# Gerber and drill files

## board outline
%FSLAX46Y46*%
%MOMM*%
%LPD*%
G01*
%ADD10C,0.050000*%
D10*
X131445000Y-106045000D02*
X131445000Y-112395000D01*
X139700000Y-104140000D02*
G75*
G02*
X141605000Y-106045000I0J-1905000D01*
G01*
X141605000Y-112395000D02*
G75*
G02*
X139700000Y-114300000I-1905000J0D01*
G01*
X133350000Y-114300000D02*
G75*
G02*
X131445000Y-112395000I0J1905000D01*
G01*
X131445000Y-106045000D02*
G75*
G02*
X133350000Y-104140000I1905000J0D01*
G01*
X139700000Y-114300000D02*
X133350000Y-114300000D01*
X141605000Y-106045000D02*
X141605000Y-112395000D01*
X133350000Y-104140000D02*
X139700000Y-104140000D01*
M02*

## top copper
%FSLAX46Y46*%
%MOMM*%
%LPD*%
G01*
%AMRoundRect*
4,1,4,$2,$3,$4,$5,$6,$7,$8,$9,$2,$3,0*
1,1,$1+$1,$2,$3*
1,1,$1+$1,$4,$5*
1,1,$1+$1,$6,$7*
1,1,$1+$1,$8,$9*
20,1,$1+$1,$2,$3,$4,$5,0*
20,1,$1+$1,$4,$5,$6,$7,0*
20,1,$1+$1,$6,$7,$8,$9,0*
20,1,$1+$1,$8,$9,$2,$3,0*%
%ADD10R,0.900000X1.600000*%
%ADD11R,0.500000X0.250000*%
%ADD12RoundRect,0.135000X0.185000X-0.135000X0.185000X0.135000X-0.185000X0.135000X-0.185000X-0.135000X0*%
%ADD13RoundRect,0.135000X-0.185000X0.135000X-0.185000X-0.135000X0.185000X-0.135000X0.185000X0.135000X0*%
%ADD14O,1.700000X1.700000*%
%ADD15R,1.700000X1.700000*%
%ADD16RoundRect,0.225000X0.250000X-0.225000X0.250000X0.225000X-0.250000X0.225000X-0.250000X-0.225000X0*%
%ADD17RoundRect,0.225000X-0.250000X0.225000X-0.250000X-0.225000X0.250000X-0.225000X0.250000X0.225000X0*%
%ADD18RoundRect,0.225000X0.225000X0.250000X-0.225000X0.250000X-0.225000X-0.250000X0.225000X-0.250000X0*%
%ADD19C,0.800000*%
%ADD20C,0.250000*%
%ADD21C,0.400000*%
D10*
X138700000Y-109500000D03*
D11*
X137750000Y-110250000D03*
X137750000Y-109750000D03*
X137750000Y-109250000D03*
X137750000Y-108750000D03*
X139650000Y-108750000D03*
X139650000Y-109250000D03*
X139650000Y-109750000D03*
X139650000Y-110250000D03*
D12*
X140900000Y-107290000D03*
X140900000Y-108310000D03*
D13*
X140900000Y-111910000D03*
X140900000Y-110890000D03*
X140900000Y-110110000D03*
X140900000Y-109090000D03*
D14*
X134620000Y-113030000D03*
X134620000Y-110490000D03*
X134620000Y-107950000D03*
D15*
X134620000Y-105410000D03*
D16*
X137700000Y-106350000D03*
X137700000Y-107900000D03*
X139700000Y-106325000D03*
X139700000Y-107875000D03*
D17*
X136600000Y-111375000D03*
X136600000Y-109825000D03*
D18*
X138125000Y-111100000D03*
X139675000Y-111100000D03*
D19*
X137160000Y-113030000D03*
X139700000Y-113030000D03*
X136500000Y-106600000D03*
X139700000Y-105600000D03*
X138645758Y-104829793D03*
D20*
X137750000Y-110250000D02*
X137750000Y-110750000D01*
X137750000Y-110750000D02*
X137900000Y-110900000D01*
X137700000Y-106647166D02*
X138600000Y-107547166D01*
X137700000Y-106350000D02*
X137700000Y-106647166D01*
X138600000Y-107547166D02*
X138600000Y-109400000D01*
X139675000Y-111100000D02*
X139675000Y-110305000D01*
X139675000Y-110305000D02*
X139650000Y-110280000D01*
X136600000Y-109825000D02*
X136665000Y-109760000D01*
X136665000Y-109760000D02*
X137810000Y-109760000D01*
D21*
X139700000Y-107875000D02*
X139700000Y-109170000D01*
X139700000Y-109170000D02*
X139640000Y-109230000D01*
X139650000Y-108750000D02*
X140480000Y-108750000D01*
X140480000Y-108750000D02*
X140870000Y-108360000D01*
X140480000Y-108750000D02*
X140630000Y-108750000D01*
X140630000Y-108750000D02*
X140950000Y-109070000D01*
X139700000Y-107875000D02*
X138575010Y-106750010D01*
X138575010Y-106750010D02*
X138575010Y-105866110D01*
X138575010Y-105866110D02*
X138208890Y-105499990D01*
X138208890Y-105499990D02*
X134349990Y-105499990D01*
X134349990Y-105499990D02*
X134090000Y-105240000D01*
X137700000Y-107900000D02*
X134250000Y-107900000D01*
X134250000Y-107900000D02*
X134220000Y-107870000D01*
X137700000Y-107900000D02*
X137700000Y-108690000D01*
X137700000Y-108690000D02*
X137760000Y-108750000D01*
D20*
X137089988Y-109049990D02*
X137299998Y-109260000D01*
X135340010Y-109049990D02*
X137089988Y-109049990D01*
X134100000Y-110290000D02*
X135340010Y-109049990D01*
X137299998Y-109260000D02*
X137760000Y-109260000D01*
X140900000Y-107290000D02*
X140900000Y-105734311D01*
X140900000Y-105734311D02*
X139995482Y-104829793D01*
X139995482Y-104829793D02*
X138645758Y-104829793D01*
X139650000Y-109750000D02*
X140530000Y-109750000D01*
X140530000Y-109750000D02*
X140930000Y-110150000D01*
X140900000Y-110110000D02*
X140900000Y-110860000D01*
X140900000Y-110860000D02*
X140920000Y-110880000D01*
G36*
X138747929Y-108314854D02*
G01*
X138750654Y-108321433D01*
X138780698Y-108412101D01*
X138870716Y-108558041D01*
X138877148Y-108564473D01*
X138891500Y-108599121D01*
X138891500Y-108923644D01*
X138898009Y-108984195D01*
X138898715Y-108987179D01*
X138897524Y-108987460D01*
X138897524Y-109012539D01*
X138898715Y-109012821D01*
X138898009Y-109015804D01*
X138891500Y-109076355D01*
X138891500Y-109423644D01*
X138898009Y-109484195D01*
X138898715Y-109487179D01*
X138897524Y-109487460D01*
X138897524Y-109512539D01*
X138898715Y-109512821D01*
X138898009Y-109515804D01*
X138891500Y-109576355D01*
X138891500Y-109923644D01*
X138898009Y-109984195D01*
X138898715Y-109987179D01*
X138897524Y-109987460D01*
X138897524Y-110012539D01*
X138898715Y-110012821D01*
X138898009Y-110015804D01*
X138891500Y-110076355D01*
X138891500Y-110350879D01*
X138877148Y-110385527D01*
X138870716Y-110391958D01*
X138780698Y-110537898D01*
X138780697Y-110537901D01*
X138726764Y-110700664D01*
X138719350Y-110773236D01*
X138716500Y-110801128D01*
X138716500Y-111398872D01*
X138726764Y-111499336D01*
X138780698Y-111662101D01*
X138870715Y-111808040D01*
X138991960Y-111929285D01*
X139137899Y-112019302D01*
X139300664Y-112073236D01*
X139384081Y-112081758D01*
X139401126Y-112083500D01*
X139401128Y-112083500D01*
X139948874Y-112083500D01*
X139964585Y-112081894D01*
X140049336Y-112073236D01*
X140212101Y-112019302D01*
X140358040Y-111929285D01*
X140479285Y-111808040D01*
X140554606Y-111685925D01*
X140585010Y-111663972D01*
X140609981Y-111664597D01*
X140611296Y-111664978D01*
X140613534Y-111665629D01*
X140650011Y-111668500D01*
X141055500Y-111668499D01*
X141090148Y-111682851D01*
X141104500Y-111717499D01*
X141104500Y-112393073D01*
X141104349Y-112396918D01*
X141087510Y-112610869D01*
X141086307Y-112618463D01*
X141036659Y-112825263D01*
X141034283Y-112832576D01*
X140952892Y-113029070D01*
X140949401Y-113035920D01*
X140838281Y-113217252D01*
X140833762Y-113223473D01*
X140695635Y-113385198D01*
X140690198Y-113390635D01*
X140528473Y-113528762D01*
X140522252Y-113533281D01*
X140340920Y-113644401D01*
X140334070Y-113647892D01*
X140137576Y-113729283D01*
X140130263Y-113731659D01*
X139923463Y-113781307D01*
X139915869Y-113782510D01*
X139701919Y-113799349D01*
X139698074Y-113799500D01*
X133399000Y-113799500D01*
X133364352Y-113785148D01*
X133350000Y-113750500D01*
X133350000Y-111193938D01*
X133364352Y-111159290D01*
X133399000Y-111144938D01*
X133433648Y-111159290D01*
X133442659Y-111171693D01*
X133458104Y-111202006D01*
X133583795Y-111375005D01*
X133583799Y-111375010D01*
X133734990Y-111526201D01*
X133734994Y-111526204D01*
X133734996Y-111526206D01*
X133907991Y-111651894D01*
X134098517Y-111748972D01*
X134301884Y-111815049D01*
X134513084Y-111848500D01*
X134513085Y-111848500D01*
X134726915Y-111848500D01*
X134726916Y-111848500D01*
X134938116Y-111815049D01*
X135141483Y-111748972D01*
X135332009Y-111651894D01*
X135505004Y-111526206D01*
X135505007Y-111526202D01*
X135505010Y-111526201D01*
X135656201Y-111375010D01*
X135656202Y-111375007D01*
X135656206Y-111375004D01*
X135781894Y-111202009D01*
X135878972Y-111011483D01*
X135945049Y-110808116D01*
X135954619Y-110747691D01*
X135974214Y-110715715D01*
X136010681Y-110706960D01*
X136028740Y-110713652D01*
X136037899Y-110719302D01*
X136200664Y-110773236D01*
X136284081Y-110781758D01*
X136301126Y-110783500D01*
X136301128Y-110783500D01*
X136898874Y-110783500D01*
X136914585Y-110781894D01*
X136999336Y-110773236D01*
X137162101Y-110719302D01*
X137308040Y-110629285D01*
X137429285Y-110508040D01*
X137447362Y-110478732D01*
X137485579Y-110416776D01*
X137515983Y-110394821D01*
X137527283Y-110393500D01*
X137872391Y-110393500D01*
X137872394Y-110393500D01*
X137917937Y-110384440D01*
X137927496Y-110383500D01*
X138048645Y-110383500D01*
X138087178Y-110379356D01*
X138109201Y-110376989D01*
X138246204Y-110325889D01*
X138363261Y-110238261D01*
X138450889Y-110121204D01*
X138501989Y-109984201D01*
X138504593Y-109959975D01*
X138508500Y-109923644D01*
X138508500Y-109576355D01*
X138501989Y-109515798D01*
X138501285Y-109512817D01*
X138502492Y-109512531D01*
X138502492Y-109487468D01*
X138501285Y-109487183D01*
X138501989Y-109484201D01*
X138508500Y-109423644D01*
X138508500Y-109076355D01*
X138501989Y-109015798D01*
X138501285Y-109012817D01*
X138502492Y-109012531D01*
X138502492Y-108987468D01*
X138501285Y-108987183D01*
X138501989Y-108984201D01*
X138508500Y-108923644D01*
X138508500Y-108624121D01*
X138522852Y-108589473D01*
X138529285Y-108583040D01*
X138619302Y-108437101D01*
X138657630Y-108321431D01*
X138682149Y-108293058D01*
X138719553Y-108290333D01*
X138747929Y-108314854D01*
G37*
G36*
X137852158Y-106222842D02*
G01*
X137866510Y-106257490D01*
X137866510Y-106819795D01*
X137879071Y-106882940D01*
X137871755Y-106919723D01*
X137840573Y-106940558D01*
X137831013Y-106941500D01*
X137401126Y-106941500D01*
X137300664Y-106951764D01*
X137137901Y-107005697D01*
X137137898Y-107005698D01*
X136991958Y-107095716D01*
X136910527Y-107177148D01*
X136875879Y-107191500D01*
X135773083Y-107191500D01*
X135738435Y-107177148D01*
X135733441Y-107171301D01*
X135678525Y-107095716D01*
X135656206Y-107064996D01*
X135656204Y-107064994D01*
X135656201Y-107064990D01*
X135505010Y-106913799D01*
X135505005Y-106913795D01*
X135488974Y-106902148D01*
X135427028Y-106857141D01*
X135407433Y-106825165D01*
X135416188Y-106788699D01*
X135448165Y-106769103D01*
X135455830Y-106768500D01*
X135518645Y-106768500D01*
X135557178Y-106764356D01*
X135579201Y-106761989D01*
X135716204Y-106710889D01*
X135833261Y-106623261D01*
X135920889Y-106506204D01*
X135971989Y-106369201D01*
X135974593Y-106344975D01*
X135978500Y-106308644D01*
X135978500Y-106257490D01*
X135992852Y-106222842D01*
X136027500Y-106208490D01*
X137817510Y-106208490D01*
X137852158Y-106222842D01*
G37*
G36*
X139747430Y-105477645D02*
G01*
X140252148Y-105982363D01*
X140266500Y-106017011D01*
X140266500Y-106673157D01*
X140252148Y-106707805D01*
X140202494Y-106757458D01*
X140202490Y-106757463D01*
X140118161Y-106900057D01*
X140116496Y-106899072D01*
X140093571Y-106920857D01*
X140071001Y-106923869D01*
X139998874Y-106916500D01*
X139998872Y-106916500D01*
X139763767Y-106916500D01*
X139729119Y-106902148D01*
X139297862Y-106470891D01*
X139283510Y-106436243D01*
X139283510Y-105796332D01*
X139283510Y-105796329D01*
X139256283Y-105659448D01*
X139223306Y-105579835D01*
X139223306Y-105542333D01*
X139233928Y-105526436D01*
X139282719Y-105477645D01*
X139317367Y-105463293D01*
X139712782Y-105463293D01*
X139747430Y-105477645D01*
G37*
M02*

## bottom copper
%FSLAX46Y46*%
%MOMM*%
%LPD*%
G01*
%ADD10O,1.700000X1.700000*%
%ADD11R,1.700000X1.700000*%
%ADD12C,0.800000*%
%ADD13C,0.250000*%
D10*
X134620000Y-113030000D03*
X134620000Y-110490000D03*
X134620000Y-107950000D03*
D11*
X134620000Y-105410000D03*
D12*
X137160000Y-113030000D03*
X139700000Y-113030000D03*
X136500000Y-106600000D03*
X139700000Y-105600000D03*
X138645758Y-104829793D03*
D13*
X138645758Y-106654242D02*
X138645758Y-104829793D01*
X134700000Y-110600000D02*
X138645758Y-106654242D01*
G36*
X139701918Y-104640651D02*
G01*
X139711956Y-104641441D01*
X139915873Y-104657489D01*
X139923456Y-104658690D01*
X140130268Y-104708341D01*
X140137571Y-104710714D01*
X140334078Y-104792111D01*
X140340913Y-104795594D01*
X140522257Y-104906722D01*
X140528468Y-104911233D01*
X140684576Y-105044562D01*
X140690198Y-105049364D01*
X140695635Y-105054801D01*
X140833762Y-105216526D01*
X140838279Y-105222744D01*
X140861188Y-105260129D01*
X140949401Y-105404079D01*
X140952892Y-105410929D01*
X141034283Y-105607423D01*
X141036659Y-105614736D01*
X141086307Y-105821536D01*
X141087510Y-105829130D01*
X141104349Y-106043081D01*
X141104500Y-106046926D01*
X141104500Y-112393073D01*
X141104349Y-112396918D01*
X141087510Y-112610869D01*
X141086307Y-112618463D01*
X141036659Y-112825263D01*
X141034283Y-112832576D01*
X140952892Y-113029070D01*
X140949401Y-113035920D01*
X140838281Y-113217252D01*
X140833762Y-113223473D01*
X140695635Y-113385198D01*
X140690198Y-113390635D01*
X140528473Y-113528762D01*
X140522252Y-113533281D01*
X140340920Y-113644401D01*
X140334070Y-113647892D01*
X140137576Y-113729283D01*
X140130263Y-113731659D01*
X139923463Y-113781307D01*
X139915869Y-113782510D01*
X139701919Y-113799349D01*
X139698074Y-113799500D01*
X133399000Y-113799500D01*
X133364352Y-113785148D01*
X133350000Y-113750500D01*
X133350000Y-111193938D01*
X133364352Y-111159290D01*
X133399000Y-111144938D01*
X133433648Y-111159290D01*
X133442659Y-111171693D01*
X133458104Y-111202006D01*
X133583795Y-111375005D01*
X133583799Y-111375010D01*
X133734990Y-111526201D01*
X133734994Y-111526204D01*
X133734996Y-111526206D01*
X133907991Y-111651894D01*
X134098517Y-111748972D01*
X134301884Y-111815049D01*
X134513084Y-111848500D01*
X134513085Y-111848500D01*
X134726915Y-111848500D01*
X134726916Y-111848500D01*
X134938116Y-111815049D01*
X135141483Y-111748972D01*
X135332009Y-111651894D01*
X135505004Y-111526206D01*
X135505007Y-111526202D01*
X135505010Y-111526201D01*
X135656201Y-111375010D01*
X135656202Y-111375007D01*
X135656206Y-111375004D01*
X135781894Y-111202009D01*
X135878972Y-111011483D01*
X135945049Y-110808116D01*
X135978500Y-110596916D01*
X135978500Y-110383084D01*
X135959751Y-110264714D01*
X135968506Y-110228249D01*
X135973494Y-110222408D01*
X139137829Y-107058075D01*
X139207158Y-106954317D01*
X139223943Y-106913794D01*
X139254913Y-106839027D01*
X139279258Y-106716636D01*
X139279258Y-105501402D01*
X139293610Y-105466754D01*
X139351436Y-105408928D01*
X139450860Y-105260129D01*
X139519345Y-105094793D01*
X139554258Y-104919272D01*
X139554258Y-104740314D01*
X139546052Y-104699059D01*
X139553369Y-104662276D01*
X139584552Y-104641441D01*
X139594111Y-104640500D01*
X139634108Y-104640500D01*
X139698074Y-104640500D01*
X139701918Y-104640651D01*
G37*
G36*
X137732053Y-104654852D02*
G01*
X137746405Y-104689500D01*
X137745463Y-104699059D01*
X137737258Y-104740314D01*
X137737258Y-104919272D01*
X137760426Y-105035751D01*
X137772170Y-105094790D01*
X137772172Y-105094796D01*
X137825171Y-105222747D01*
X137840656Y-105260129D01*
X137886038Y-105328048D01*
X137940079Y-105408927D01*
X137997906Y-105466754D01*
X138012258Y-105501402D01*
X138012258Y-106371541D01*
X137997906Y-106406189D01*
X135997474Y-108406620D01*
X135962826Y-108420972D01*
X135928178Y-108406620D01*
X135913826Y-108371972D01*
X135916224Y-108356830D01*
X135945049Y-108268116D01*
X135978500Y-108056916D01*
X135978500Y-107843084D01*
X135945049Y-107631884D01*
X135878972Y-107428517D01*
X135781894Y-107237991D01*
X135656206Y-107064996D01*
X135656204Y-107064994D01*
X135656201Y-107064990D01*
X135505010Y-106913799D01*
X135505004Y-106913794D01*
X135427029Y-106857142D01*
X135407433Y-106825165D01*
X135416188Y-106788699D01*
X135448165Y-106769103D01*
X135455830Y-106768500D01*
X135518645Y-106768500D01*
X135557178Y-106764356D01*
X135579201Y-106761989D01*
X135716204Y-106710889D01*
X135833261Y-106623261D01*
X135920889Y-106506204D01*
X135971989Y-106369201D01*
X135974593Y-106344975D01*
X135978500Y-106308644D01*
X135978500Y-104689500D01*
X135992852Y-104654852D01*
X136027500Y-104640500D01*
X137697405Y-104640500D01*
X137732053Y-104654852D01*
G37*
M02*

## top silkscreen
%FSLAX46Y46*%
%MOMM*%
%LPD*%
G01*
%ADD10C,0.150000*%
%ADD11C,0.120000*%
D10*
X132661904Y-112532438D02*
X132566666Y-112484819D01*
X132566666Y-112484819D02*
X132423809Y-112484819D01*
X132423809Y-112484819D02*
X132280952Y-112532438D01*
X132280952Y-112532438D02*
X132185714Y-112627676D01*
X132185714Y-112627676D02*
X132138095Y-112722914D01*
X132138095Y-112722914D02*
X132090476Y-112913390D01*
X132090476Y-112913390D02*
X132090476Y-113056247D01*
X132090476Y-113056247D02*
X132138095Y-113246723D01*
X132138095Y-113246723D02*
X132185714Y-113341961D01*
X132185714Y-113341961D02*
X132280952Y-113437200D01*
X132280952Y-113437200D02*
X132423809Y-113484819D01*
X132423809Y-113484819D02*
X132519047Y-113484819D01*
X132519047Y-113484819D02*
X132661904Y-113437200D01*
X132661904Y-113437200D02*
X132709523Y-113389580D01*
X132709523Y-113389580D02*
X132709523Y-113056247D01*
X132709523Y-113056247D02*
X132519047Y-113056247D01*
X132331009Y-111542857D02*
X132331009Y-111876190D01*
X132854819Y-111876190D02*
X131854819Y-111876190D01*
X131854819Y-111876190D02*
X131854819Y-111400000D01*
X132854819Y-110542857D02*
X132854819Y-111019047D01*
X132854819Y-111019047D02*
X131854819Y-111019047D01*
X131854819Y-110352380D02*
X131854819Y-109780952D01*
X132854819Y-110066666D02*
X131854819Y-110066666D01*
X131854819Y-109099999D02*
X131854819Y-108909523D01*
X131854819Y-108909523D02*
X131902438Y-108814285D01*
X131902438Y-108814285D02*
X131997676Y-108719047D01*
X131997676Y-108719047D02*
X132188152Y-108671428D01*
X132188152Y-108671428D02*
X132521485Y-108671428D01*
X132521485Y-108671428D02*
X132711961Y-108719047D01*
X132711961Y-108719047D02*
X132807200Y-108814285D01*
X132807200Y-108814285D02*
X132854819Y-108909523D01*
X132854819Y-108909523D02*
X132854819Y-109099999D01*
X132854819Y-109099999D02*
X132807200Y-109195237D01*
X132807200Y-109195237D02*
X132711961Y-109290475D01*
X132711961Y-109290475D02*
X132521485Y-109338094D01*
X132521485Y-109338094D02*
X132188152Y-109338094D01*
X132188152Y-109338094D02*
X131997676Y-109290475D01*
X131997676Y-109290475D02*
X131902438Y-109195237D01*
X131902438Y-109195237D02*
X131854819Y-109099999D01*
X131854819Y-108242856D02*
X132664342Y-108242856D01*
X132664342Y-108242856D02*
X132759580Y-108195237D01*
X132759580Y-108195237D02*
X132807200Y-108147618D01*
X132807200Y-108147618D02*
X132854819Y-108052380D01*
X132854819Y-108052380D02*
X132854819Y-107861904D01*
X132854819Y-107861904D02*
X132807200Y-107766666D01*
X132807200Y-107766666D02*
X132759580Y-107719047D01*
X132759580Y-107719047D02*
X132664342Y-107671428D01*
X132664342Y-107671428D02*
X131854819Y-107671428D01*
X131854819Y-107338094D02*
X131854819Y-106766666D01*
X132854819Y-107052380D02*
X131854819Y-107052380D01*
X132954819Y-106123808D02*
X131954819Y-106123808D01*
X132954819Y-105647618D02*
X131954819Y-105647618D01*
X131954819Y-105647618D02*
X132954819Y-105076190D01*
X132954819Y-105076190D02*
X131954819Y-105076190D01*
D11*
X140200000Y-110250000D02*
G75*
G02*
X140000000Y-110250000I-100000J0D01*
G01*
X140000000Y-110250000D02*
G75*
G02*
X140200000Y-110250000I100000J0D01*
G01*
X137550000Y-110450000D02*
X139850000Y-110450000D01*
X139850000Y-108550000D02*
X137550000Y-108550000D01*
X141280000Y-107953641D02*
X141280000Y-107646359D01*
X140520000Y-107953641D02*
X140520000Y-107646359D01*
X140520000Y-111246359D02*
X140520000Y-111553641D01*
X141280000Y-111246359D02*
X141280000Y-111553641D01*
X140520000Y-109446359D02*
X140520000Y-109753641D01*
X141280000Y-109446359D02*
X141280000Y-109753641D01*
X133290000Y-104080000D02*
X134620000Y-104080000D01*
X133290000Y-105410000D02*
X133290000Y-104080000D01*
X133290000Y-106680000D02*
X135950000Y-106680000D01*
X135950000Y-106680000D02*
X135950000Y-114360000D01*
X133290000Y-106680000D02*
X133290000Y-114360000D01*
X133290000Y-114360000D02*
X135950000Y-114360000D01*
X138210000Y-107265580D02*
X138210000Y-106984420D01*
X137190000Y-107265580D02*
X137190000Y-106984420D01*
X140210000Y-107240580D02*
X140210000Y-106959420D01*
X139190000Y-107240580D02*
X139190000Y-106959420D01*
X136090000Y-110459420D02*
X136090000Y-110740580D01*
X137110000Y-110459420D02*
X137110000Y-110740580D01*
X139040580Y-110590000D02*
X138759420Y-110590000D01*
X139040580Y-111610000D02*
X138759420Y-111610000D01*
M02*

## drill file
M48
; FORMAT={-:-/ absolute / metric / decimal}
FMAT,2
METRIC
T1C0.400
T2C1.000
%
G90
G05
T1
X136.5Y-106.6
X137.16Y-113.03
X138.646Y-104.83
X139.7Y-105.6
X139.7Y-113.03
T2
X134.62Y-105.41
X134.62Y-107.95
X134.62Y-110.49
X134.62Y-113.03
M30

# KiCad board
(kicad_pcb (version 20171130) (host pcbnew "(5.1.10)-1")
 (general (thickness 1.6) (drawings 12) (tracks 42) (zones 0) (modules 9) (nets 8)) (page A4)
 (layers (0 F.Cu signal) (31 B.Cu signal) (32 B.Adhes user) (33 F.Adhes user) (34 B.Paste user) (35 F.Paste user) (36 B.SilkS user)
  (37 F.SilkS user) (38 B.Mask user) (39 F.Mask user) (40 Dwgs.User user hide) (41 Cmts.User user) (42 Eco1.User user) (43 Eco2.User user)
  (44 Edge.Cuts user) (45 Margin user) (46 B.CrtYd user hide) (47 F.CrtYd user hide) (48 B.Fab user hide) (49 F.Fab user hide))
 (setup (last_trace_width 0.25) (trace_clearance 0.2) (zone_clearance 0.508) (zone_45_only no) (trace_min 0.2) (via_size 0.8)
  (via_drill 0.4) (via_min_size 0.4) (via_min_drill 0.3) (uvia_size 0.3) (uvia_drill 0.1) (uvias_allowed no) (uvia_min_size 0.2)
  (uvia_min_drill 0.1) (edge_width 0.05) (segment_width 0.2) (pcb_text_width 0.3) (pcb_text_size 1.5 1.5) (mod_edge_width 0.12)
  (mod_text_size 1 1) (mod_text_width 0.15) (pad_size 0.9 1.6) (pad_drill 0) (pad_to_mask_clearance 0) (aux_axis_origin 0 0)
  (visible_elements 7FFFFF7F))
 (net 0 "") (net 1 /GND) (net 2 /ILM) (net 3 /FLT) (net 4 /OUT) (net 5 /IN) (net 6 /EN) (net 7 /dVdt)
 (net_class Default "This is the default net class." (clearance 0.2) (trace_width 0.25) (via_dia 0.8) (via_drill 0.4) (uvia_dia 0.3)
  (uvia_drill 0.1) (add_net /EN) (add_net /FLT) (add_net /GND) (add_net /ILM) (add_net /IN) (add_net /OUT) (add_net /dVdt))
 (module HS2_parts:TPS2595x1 (layer F.Cu) (at 138.7 109.5 180)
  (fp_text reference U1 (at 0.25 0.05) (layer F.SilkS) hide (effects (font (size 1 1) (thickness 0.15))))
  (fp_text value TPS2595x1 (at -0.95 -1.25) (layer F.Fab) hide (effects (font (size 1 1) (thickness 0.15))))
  (fp_circle (center -1.4 -0.75) (end -1.3 -0.75) (layer F.SilkS) (width 0.12))
  (fp_line (start 1.15 -0.95) (end -1.15 -0.95) (layer F.SilkS) (width 0.12))
  (fp_line (start -1.15 0.95) (end 1.15 0.95) (layer F.SilkS) (width 0.12))
  (pad 8 smd rect (at 0 0 180) (size 0.9 1.6) (layers F.Cu F.Paste F.Mask) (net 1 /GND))
  (pad 8 smd rect (at 0.95 -0.75 180) (size 0.5 0.25) (layers F.Cu F.Paste F.Mask) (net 1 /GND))
  (pad 7 smd rect (at 0.95 -0.25 180) (size 0.5 0.25) (layers F.Cu F.Paste F.Mask) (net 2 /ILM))
  (pad 6 smd rect (at 0.95 0.25 180) (size 0.5 0.25) (layers F.Cu F.Paste F.Mask) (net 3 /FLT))
  (pad 5 smd rect (at 0.95 0.75 180) (size 0.5 0.25) (layers F.Cu F.Paste F.Mask) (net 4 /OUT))
  (pad 4 smd rect (at -0.95 0.75 180) (size 0.5 0.25) (layers F.Cu F.Paste F.Mask) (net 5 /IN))
  (pad 3 smd rect (at -0.95 0.25 180) (size 0.5 0.25) (layers F.Cu F.Paste F.Mask) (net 5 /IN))
  (pad 2 smd rect (at -0.95 -0.25 180) (size 0.5 0.25) (layers F.Cu F.Paste F.Mask) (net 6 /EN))
  (pad 1 smd rect (at -0.95 -0.75 180) (size 0.5 0.25) (layers F.Cu F.Paste F.Mask) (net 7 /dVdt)))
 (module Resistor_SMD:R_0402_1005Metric (layer F.Cu) (at 140.9 107.8 90)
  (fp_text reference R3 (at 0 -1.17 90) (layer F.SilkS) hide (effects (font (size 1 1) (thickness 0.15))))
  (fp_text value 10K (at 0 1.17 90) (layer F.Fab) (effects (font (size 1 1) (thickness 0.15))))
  (fp_line (start -0.153641 0.38) (end 0.153641 0.38) (layer F.SilkS) (width 0.12))
  (fp_line (start -0.153641 -0.38) (end 0.153641 -0.38) (layer F.SilkS) (width 0.12))
  (pad 2 smd roundrect (at 0.51 0 90) (size 0.54 0.64) (layers F.Cu F.Paste F.Mask) (roundrect_rratio 0.25) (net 3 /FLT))
  (pad 1 smd roundrect (at -0.51 0 90) (size 0.54 0.64) (layers F.Cu F.Paste F.Mask) (roundrect_rratio 0.25) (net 5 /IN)))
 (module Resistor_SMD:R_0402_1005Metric (layer F.Cu) (at 140.9 111.4 270)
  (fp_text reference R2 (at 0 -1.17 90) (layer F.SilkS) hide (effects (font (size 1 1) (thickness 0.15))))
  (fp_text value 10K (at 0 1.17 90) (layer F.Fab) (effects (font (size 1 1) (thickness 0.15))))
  (fp_line (start -0.153641 0.38) (end 0.153641 0.38) (layer F.SilkS) (width 0.12))
  (fp_line (start -0.153641 -0.38) (end 0.153641 -0.38) (layer F.SilkS) (width 0.12))
  (pad 2 smd roundrect (at 0.51 0 270) (size 0.54 0.64) (layers F.Cu F.Paste F.Mask) (roundrect_rratio 0.25) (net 1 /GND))
  (pad 1 smd roundrect (at -0.51 0 270) (size 0.54 0.64) (layers F.Cu F.Paste F.Mask) (roundrect_rratio 0.25) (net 6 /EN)))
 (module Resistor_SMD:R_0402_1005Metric (layer F.Cu) (at 140.9 109.6 270)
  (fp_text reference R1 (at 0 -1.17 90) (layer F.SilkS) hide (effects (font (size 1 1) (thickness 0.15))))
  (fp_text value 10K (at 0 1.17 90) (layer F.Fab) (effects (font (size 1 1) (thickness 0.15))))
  (fp_line (start -0.153641 0.38) (end 0.153641 0.38) (layer F.SilkS) (width 0.12))
  (fp_line (start -0.153641 -0.38) (end 0.153641 -0.38) (layer F.SilkS) (width 0.12))
  (pad 2 smd roundrect (at 0.51 0 270) (size 0.54 0.64) (layers F.Cu F.Paste F.Mask) (roundrect_rratio 0.25) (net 6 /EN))
  (pad 1 smd roundrect (at -0.51 0 270) (size 0.54 0.64) (layers F.Cu F.Paste F.Mask) (roundrect_rratio 0.25) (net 5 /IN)))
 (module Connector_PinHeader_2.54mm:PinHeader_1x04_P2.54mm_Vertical (layer F.Cu) (at 134.62 105.41)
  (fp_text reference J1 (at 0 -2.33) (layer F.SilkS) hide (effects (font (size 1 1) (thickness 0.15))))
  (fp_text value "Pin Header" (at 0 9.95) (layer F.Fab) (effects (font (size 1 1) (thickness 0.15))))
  (fp_line (start -1.33 -1.33) (end 0 -1.33) (layer F.SilkS) (width 0.12))
  (fp_line (start -1.33 0) (end -1.33 -1.33) (layer F.SilkS) (width 0.12))
  (fp_line (start -1.33 1.27) (end 1.33 1.27) (layer F.SilkS) (width 0.12))
  (fp_line (start 1.33 1.27) (end 1.33 8.95) (layer F.SilkS) (width 0.12))
  (fp_line (start -1.33 1.27) (end -1.33 8.95) (layer F.SilkS) (width 0.12))
  (fp_line (start -1.33 8.95) (end 1.33 8.95) (layer F.SilkS) (width 0.12))
  (pad 4 thru_hole oval (at 0 7.62) (size 1.7 1.7) (drill 1) (layers *.Cu *.Mask) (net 1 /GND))
  (pad 3 thru_hole oval (at 0 5.08) (size 1.7 1.7) (drill 1) (layers *.Cu *.Mask) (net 3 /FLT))
  (pad 2 thru_hole oval (at 0 2.54) (size 1.7 1.7) (drill 1) (layers *.Cu *.Mask) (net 4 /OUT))
  (pad 1 thru_hole rect (at 0 0) (size 1.7 1.7) (drill 1) (layers *.Cu *.Mask) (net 5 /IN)))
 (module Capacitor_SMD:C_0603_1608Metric (layer F.Cu) (at 137.7 107.125 90)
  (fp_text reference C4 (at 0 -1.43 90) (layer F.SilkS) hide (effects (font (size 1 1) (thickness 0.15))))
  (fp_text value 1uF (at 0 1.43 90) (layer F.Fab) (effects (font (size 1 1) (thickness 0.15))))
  (fp_line (start -0.14058 0.51) (end 0.14058 0.51) (layer F.SilkS) (width 0.12))
  (fp_line (start -0.14058 -0.51) (end 0.14058 -0.51) (layer F.SilkS) (width 0.12))
  (pad 2 smd roundrect (at 0.775 0 90) (size 0.9 0.95) (layers F.Cu F.Paste F.Mask) (roundrect_rratio 0.25) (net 1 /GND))
  (pad 1 smd roundrect (at -0.775 0 90) (size 0.9 0.95) (layers F.Cu F.Paste F.Mask) (roundrect_rratio 0.25) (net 4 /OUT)))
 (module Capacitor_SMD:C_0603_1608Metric (layer F.Cu) (at 139.7 107.1 90)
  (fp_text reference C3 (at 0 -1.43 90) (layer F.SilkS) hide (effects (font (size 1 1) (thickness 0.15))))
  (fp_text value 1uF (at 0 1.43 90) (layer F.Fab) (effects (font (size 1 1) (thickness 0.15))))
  (fp_line (start -0.14058 0.51) (end 0.14058 0.51) (layer F.SilkS) (width 0.12))
  (fp_line (start -0.14058 -0.51) (end 0.14058 -0.51) (layer F.SilkS) (width 0.12))
  (pad 2 smd roundrect (at 0.775 0 90) (size 0.9 0.95) (layers F.Cu F.Paste F.Mask) (roundrect_rratio 0.25) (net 1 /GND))
  (pad 1 smd roundrect (at -0.775 0 90) (size 0.9 0.95) (layers F.Cu F.Paste F.Mask) (roundrect_rratio 0.25) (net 5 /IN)))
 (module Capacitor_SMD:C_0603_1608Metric (layer F.Cu) (at 136.6 110.6 270)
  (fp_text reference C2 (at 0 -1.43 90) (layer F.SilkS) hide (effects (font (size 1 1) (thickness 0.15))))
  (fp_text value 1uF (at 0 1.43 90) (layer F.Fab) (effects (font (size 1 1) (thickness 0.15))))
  (fp_line (start -0.14058 0.51) (end 0.14058 0.51) (layer F.SilkS) (width 0.12))
  (fp_line (start -0.14058 -0.51) (end 0.14058 -0.51) (layer F.SilkS) (width 0.12))
  (pad 2 smd roundrect (at 0.775 0 270) (size 0.9 0.95) (layers F.Cu F.Paste F.Mask) (roundrect_rratio 0.25) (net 1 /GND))
  (pad 1 smd roundrect (at -0.775 0 270) (size 0.9 0.95) (layers F.Cu F.Paste F.Mask) (roundrect_rratio 0.25) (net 2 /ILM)))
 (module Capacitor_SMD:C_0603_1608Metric (layer F.Cu) (at 138.9 111.1 180)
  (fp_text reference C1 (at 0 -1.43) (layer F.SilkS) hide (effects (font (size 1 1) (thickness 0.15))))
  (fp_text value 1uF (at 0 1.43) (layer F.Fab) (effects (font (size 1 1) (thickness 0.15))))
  (fp_line (start -0.14058 0.51) (end 0.14058 0.51) (layer F.SilkS) (width 0.12))
  (fp_line (start -0.14058 -0.51) (end 0.14058 -0.51) (layer F.SilkS) (width 0.12))
  (pad 2 smd roundrect (at 0.775 0 180) (size 0.9 0.95) (layers F.Cu F.Paste F.Mask) (roundrect_rratio 0.25) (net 1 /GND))
  (pad 1 smd roundrect (at -0.775 0 180) (size 0.9 0.95) (layers F.Cu F.Paste F.Mask) (roundrect_rratio 0.25) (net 7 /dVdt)))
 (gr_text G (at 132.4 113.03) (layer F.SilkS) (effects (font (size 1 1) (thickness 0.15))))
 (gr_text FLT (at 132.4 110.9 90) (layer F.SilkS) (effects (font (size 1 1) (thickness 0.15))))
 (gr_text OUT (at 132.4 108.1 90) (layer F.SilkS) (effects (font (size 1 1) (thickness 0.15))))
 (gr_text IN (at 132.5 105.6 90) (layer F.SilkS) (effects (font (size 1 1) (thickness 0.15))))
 (gr_line (start 131.445 106.045) (end 131.445 112.395) (layer Edge.Cuts) (width 0.05))
 (gr_arc (start 139.7 106.045) (end 141.605 106.045) (angle -90) (layer Edge.Cuts) (width 0.05))
 (gr_arc (start 139.7 112.395) (end 139.7 114.3) (angle -90) (layer Edge.Cuts) (width 0.05))
 (gr_arc (start 133.35 112.395) (end 131.445 112.395) (angle -90) (layer Edge.Cuts) (width 0.05))
 (gr_arc (start 133.35 106.045) (end 133.35 104.14) (angle -90) (layer Edge.Cuts) (width 0.05))
 (gr_line (start 139.7 114.3) (end 133.35 114.3) (layer Edge.Cuts) (width 0.05))
 (gr_line (start 141.605 106.045) (end 141.605 112.395) (layer Edge.Cuts) (width 0.05))
 (gr_line (start 133.35 104.14) (end 139.7 104.14) (layer Edge.Cuts) (width 0.05))
 (via (at 137.16 113.03) (size 0.8) (drill 0.4) (layers F.Cu B.Cu) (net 1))
 (via (at 139.7 113.03) (size 0.8) (drill 0.4) (layers F.Cu B.Cu) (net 1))
 (via (at 136.5 106.6) (size 0.8) (drill 0.4) (layers F.Cu B.Cu) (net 1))
 (segment (start 137.75 110.25) (end 137.75 110.75) (width 0.25) (layer F.Cu) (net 1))
 (segment (start 137.75 110.75) (end 137.9 110.9) (width 0.25) (layer F.Cu) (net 1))
 (via (at 139.7 105.6) (size 0.8) (drill 0.4) (layers F.Cu B.Cu) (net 1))
 (segment (start 137.7 106.647166) (end 138.6 107.547166) (width 0.25) (layer F.Cu) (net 1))
 (segment (start 137.7 106.35) (end 137.7 106.647166) (width 0.25) (layer F.Cu) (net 1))
 (segment (start 138.6 107.547166) (end 138.6 109.4) (width 0.25) (layer F.Cu) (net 1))
 (segment (start 139.675 111.1) (end 139.675 110.305) (width 0.25) (layer F.Cu) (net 7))
 (segment (start 139.675 110.305) (end 139.65 110.28) (width 0.25) (layer F.Cu) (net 7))
 (segment (start 136.6 109.825) (end 136.665 109.76) (width 0.25) (layer F.Cu) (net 2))
 (segment (start 136.665 109.76) (end 137.81 109.76) (width 0.25) (layer F.Cu) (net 2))
 (segment (start 139.7 107.875) (end 139.7 109.17) (width 0.4) (layer F.Cu) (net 5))
 (segment (start 139.7 109.17) (end 139.64 109.23) (width 0.4) (layer F.Cu) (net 5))
 (segment (start 139.65 108.75) (end 140.48 108.75) (width 0.4) (layer F.Cu) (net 5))
 (segment (start 140.48 108.75) (end 140.87 108.36) (width 0.4) (layer F.Cu) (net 5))
 (segment (start 140.48 108.75) (end 140.63 108.75) (width 0.4) (layer F.Cu) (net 5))
 (segment (start 140.63 108.75) (end 140.95 109.07) (width 0.4) (layer F.Cu) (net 5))
 (segment (start 139.7 107.875) (end 138.57501 106.75001) (width 0.4) (layer F.Cu) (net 5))
 (segment (start 138.57501 106.75001) (end 138.57501 105.86611) (width 0.4) (layer F.Cu) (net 5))
 (segment (start 138.57501 105.86611) (end 138.20889 105.49999) (width 0.4) (layer F.Cu) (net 5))
 (segment (start 138.20889 105.49999) (end 134.34999 105.49999) (width 0.4) (layer F.Cu) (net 5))
 (segment (start 134.34999 105.49999) (end 134.09 105.24) (width 0.4) (layer F.Cu) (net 5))
 (segment (start 137.7 107.9) (end 134.25 107.9) (width 0.4) (layer F.Cu) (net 4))
 (segment (start 134.25 107.9) (end 134.22 107.87) (width 0.4) (layer F.Cu) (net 4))
 (segment (start 137.7 107.9) (end 137.7 108.69) (width 0.4) (layer F.Cu) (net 4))
 (segment (start 137.7 108.69) (end 137.76 108.75) (width 0.4) (layer F.Cu) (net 4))
 (segment (start 137.089988 109.04999) (end 137.299998 109.26) (width 0.25) (layer F.Cu) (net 3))
 (segment (start 135.34001 109.04999) (end 137.089988 109.04999) (width 0.25) (layer F.Cu) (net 3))
 (segment (start 134.1 110.29) (end 135.34001 109.04999) (width 0.25) (layer F.Cu) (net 3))
 (segment (start 137.299998 109.26) (end 137.76 109.26) (width 0.25) (layer F.Cu) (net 3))
 (segment (start 140.9 107.29) (end 140.9 105.734311) (width 0.25) (layer F.Cu) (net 3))
 (via (at 138.645758 104.829793) (size 0.8) (drill 0.4) (layers F.Cu B.Cu) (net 3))
 (segment (start 138.645758 106.654242) (end 138.645758 104.829793) (width 0.25) (layer B.Cu) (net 3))
 (segment (start 140.9 105.734311) (end 139.995482 104.829793) (width 0.25) (layer F.Cu) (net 3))
 (segment (start 139.995482 104.829793) (end 138.645758 104.829793) (width 0.25) (layer F.Cu) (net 3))
 (segment (start 134.7 110.6) (end 138.645758 106.654242) (width 0.25) (layer B.Cu) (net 3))
 (segment (start 139.65 109.75) (end 140.53 109.75) (width 0.25) (layer F.Cu) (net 6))
 (segment (start 140.53 109.75) (end 140.93 110.15) (width 0.25) (layer F.Cu) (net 6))
 (segment (start 140.9 110.11) (end 140.9 110.86) (width 0.25) (layer F.Cu) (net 6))
 (segment (start 140.9 110.86) (end 140.92 110.88) (width 0.25) (layer F.Cu) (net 6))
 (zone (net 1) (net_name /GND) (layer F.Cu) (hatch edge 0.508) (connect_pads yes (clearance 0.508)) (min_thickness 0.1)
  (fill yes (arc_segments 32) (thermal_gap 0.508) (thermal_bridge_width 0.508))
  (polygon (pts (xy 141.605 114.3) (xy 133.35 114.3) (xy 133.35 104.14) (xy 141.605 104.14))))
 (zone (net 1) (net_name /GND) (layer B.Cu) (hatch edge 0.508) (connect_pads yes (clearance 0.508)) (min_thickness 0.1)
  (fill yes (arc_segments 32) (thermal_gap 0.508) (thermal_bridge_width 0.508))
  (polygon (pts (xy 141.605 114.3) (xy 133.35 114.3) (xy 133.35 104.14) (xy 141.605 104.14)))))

